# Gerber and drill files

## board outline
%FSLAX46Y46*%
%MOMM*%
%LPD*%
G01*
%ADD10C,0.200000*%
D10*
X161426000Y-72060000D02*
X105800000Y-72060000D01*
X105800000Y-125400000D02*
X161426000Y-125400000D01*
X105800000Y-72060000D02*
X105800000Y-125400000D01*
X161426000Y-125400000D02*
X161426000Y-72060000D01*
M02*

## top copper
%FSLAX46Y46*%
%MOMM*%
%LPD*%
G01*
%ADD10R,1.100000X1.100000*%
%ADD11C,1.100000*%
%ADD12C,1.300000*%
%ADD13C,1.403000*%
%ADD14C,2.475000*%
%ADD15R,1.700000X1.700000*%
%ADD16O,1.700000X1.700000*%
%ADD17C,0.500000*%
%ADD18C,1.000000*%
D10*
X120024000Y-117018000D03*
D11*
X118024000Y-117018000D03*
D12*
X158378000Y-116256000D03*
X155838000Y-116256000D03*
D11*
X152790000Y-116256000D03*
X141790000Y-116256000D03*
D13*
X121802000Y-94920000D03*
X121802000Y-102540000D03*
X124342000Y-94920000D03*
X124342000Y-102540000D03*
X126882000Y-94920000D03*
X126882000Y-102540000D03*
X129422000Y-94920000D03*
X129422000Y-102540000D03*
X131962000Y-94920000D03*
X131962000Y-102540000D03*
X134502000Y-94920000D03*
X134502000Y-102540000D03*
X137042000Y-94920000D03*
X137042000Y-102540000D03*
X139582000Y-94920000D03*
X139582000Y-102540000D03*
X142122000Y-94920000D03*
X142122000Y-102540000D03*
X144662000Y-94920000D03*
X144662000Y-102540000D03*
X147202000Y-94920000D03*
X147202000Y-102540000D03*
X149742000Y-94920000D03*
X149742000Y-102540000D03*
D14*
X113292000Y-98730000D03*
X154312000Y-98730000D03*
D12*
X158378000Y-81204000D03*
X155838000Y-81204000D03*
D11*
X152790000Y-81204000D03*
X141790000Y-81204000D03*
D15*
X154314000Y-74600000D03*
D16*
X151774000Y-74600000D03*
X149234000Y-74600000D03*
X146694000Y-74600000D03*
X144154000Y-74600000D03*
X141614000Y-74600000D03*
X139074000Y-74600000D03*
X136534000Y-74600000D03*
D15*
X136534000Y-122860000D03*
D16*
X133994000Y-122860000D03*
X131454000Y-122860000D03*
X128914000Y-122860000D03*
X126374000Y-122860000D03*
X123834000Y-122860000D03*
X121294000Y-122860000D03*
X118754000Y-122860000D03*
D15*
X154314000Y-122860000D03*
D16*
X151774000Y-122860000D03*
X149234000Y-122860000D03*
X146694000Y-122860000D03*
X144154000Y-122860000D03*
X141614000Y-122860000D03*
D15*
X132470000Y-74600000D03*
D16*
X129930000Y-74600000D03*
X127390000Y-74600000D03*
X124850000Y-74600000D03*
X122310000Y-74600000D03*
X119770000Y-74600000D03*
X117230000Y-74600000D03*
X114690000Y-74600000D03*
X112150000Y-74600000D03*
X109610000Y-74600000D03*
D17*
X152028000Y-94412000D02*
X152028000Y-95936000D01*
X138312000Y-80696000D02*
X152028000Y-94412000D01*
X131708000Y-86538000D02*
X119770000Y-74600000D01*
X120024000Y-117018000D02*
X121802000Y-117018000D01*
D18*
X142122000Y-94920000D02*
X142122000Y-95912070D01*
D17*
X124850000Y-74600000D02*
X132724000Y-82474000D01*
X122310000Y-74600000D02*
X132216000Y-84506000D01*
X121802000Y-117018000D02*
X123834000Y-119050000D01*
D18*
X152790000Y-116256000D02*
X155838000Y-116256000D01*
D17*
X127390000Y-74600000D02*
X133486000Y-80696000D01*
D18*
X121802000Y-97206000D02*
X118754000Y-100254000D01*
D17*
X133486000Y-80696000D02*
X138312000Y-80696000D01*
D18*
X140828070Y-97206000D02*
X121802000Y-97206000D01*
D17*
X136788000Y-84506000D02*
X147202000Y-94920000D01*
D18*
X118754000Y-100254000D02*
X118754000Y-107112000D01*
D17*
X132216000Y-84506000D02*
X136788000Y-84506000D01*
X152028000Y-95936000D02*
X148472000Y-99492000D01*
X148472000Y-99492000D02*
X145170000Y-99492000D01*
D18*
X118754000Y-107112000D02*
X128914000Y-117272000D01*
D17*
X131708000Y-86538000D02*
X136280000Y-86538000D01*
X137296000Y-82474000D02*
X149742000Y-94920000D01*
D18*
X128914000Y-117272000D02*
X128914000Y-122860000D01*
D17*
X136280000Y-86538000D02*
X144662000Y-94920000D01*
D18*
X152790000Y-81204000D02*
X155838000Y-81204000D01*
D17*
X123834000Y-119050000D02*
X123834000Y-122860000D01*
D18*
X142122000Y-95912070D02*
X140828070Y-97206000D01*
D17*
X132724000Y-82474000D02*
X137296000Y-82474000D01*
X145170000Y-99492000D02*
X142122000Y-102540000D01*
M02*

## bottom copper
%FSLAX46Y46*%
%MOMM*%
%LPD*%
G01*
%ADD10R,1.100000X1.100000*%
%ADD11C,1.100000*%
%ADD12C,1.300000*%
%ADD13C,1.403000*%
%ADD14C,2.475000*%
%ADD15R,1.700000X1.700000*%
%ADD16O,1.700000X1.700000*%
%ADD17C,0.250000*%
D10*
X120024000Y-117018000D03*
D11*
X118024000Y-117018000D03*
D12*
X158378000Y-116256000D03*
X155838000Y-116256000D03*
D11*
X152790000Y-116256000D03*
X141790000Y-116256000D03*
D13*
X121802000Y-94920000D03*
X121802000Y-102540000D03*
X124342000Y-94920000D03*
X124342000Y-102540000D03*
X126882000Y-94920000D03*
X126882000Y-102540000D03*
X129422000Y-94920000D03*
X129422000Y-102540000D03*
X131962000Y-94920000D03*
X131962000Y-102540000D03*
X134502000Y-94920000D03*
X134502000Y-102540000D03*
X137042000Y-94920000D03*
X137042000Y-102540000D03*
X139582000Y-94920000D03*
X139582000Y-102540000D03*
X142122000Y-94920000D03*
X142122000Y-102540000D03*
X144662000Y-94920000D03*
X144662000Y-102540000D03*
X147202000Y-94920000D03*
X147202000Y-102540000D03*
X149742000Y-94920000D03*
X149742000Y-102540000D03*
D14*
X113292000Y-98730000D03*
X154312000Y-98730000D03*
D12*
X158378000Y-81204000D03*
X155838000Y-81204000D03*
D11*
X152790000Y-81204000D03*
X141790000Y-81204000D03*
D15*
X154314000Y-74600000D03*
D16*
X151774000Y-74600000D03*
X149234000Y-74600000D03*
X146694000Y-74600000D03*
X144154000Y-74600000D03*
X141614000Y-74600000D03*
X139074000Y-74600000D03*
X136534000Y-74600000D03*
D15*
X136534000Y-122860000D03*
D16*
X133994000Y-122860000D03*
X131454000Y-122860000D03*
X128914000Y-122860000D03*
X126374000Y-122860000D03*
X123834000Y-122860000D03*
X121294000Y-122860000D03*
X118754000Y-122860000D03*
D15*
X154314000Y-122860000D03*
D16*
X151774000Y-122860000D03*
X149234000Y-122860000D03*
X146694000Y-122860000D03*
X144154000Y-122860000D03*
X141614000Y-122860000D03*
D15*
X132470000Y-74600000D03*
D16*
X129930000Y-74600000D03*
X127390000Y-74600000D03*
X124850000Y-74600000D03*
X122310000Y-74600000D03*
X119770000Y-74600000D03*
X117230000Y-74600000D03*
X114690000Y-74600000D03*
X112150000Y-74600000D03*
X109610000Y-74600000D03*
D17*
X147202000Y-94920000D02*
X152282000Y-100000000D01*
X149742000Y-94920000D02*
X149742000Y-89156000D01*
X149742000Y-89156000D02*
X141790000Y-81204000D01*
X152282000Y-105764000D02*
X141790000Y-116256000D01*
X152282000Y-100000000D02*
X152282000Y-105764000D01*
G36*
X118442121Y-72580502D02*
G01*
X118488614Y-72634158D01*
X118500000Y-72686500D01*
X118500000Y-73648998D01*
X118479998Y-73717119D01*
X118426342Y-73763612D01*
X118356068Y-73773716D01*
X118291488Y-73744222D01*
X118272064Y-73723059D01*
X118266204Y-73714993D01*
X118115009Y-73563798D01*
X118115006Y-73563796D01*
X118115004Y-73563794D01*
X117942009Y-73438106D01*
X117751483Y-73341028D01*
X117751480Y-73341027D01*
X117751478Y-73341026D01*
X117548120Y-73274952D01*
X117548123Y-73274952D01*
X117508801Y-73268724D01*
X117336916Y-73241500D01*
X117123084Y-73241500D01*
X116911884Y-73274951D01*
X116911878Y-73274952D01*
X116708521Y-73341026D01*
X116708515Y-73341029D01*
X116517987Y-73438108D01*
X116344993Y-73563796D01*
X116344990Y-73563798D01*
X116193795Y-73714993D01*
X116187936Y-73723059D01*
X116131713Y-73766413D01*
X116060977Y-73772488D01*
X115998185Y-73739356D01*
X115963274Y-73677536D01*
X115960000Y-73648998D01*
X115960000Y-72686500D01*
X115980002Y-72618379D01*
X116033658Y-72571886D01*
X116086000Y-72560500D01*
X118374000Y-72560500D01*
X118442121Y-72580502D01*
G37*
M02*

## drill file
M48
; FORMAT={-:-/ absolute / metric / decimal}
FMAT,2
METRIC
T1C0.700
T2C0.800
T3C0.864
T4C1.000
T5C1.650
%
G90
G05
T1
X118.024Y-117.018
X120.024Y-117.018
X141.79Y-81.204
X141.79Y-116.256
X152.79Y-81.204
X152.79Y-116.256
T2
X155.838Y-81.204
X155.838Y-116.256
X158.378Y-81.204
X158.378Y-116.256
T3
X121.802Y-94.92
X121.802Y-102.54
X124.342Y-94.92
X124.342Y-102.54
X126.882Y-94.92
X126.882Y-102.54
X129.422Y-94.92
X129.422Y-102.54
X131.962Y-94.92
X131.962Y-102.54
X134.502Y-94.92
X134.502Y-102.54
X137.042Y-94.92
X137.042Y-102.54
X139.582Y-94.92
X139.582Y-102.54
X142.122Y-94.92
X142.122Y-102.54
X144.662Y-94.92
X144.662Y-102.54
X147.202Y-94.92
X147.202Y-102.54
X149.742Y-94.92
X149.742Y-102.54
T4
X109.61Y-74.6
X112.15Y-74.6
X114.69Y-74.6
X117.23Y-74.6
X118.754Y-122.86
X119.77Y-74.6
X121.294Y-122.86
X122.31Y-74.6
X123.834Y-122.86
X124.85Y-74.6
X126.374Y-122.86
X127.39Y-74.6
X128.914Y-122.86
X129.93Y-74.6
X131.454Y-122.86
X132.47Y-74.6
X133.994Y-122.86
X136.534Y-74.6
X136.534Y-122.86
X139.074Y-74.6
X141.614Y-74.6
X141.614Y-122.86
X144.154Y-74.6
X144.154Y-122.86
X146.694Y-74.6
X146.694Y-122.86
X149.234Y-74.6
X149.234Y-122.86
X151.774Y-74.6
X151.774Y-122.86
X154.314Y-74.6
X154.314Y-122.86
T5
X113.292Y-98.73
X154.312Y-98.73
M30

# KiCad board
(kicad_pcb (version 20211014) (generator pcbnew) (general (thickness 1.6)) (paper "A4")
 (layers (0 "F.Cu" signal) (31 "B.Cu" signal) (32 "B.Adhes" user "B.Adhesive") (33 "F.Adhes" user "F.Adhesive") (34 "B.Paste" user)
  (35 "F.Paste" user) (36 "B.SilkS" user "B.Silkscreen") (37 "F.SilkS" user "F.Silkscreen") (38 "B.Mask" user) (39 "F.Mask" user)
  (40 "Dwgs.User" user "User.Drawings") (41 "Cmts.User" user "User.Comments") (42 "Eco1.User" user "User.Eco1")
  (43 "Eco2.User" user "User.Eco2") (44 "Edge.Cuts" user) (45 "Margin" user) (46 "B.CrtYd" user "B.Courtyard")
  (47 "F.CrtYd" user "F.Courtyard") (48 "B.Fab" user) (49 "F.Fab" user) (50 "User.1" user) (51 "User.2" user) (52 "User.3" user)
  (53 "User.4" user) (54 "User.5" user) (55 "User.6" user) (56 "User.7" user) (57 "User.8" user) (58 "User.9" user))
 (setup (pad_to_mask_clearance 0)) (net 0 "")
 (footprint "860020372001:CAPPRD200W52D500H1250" (layer "F.Cu") (at 120.024 117.018 180)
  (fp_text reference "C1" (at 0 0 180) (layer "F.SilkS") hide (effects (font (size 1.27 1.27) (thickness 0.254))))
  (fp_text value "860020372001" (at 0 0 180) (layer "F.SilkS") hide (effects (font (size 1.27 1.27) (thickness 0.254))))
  (pad "1" thru_hole rect locked (at 0 0 180) (size 1.1 1.1) (drill 0.7) (layers F&B.Cu *.Mask))
  (pad "2" thru_hole circle locked (at 2 0 180) (size 1.1 1.1) (drill 0.7) (layers F&B.Cu *.Mask)))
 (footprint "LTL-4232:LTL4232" (layer "F.Cu") (at 158.378 116.256 180)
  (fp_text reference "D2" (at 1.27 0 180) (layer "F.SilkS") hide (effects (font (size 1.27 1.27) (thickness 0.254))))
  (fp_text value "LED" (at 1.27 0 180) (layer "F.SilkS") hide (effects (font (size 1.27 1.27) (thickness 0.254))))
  (pad "1" thru_hole circle locked (at 0 0 180) (size 1.3 1.3) (drill 0.8) (layers F&B.Cu *.Mask))
  (pad "2" thru_hole circle locked (at 2.54 0 180) (size 1.3 1.3) (drill 0.8) (layers F&B.Cu *.Mask)))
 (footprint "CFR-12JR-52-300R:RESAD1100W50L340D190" (layer "F.Cu") (at 152.79 116.256 180)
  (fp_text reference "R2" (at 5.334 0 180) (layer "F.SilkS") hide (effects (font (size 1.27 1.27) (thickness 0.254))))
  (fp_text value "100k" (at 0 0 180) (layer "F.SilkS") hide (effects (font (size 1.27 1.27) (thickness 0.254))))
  (pad "1" thru_hole circle locked (at 0 0 180) (size 1.1 1.1) (drill 0.7) (layers F&B.Cu *.Mask))
  (pad "2" thru_hole circle locked (at 11 0 180) (size 1.1 1.1) (drill 0.7) (layers F&B.Cu *.Mask)))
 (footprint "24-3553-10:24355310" (layer "F.Cu") (at 121.802 94.92)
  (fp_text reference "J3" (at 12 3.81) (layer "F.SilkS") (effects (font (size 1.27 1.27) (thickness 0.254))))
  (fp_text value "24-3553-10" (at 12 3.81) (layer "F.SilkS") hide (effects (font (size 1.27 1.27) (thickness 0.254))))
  (pad "1" thru_hole circle locked (at 0 0) (size 1.403 1.403) (drill 0.8636) (layers F&B.Cu *.Mask))
  (pad "2" thru_hole circle locked (at 0 7.62) (size 1.403 1.403) (drill 0.8636) (layers F&B.Cu *.Mask))
  (pad "3" thru_hole circle locked (at 2.54 0) (size 1.403 1.403) (drill 0.8636) (layers F&B.Cu *.Mask))
  (pad "4" thru_hole circle locked (at 2.54 7.62) (size 1.403 1.403) (drill 0.8636) (layers F&B.Cu *.Mask))
  (pad "5" thru_hole circle locked (at 5.08 0) (size 1.403 1.403) (drill 0.8636) (layers F&B.Cu *.Mask))
  (pad "6" thru_hole circle locked (at 5.08 7.62) (size 1.403 1.403) (drill 0.8636) (layers F&B.Cu *.Mask))
  (pad "7" thru_hole circle locked (at 7.62 0) (size 1.403 1.403) (drill 0.8636) (layers F&B.Cu *.Mask))
  (pad "8" thru_hole circle locked (at 7.62 7.62) (size 1.403 1.403) (drill 0.8636) (layers F&B.Cu *.Mask))
  (pad "9" thru_hole circle locked (at 10.16 0) (size 1.403 1.403) (drill 0.8636) (layers F&B.Cu *.Mask))
  (pad "10" thru_hole circle locked (at 10.16 7.62) (size 1.403 1.403) (drill 0.8636) (layers F&B.Cu *.Mask))
  (pad "11" thru_hole circle locked (at 12.7 0) (size 1.403 1.403) (drill 0.8636) (layers F&B.Cu *.Mask))
  (pad "12" thru_hole circle locked (at 12.7 7.62) (size 1.403 1.403) (drill 0.8636) (layers F&B.Cu *.Mask))
  (pad "13" thru_hole circle locked (at 15.24 0) (size 1.403 1.403) (drill 0.8636) (layers F&B.Cu *.Mask))
  (pad "14" thru_hole circle locked (at 15.24 7.62) (size 1.403 1.403) (drill 0.8636) (layers F&B.Cu *.Mask))
  (pad "15" thru_hole circle locked (at 17.78 0) (size 1.403 1.403) (drill 0.8636) (layers F&B.Cu *.Mask))
  (pad "16" thru_hole circle locked (at 17.78 7.62) (size 1.403 1.403) (drill 0.8636) (layers F&B.Cu *.Mask))
  (pad "17" thru_hole circle locked (at 20.32 0) (size 1.403 1.403) (drill 0.8636) (layers F&B.Cu *.Mask))
  (pad "18" thru_hole circle locked (at 20.32 7.62) (size 1.403 1.403) (drill 0.8636) (layers F&B.Cu *.Mask))
  (pad "19" thru_hole circle locked (at 22.86 0) (size 1.403 1.403) (drill 0.8636) (layers F&B.Cu *.Mask))
  (pad "20" thru_hole circle locked (at 22.86 7.62) (size 1.403 1.403) (drill 0.8636) (layers F&B.Cu *.Mask))
  (pad "21" thru_hole circle locked (at 25.4 0) (size 1.403 1.403) (drill 0.8636) (layers F&B.Cu *.Mask))
  (pad "22" thru_hole circle locked (at 25.4 7.62) (size 1.403 1.403) (drill 0.8636) (layers F&B.Cu *.Mask))
  (pad "23" thru_hole circle locked (at 27.94 0) (size 1.403 1.403) (drill 0.8636) (layers F&B.Cu *.Mask))
  (pad "24" thru_hole circle locked (at 27.94 7.62) (size 1.403 1.403) (drill 0.8636) (layers F&B.Cu *.Mask))
  (pad "MH1" thru_hole circle locked (at -8.51 3.81) (size 2.475 2.475) (drill 1.65) (layers F&B.Cu *.Mask))
  (pad "MH2" thru_hole circle locked (at 32.51 3.81) (size 2.475 2.475) (drill 1.65) (layers F&B.Cu *.Mask)))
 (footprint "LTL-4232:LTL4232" (layer "F.Cu") (at 158.378 81.204 180)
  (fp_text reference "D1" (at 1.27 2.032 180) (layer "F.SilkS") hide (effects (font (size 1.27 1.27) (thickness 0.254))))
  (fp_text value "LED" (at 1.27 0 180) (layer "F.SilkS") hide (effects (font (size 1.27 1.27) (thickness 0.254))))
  (pad "1" thru_hole circle locked (at 0 0 180) (size 1.3 1.3) (drill 0.8) (layers F&B.Cu *.Mask))
  (pad "2" thru_hole circle locked (at 2.54 0 180) (size 1.3 1.3) (drill 0.8) (layers F&B.Cu *.Mask)))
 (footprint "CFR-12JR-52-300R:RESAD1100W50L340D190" (layer "F.Cu") (at 152.79 81.204 180)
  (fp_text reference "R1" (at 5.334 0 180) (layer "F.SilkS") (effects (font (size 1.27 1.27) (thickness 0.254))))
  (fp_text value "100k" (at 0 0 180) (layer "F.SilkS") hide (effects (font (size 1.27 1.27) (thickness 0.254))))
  (pad "1" thru_hole circle locked (at 0 0 180) (size 1.1 1.1) (drill 0.7) (layers F&B.Cu *.Mask))
  (pad "2" thru_hole circle locked (at 11 0 180) (size 1.1 1.1) (drill 0.7) (layers F&B.Cu *.Mask)))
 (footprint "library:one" (layer "B.Cu") (at 135.01 90.094)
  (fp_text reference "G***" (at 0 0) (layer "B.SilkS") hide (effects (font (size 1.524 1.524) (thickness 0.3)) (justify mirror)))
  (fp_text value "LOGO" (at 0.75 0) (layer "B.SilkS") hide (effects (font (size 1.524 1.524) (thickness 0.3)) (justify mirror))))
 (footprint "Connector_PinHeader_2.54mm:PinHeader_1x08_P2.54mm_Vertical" (layer "B.Cu") (at 154.314 74.6 90)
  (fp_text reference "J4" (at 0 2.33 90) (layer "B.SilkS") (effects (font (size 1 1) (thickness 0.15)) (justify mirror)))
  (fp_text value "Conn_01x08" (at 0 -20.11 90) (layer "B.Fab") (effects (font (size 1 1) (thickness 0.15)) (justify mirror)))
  (pad "1" thru_hole rect locked (at 0 0 90) (size 1.7 1.7) (drill 1) (layers F&B.Cu *.Mask))
  (pad "2" thru_hole oval locked (at 0 -2.54 90) (size 1.7 1.7) (drill 1) (layers F&B.Cu *.Mask))
  (pad "3" thru_hole oval locked (at 0 -5.08 90) (size 1.7 1.7) (drill 1) (layers F&B.Cu *.Mask))
  (pad "4" thru_hole oval locked (at 0 -7.62 90) (size 1.7 1.7) (drill 1) (layers F&B.Cu *.Mask))
  (pad "5" thru_hole oval locked (at 0 -10.16 90) (size 1.7 1.7) (drill 1) (layers F&B.Cu *.Mask))
  (pad "6" thru_hole oval locked (at 0 -12.7 90) (size 1.7 1.7) (drill 1) (layers F&B.Cu *.Mask))
  (pad "7" thru_hole oval locked (at 0 -15.24 90) (size 1.7 1.7) (drill 1) (layers F&B.Cu *.Mask))
  (pad "8" thru_hole oval locked (at 0 -17.78 90) (size 1.7 1.7) (drill 1) (layers F&B.Cu *.Mask)))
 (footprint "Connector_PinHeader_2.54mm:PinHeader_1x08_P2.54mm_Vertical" (layer "B.Cu") (at 136.534 122.86 90)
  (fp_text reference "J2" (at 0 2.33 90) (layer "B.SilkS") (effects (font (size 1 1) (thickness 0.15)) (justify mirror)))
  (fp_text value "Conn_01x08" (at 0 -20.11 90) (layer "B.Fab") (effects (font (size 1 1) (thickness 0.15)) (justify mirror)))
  (pad "1" thru_hole rect locked (at 0 0 90) (size 1.7 1.7) (drill 1) (layers F&B.Cu *.Mask))
  (pad "2" thru_hole oval locked (at 0 -2.54 90) (size 1.7 1.7) (drill 1) (layers F&B.Cu *.Mask))
  (pad "3" thru_hole oval locked (at 0 -5.08 90) (size 1.7 1.7) (drill 1) (layers F&B.Cu *.Mask))
  (pad "4" thru_hole oval locked (at 0 -7.62 90) (size 1.7 1.7) (drill 1) (layers F&B.Cu *.Mask))
  (pad "5" thru_hole oval locked (at 0 -10.16 90) (size 1.7 1.7) (drill 1) (layers F&B.Cu *.Mask))
  (pad "6" thru_hole oval locked (at 0 -12.7 90) (size 1.7 1.7) (drill 1) (layers F&B.Cu *.Mask))
  (pad "7" thru_hole oval locked (at 0 -15.24 90) (size 1.7 1.7) (drill 1) (layers F&B.Cu *.Mask))
  (pad "8" thru_hole oval locked (at 0 -17.78 90) (size 1.7 1.7) (drill 1) (layers F&B.Cu *.Mask)))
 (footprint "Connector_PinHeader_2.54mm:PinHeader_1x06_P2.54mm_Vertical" (layer "B.Cu") (at 154.314 122.86 90)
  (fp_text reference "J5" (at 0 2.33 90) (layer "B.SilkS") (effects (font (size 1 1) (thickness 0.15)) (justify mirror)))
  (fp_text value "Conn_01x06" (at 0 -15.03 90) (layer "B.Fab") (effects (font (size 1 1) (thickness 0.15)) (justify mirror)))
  (pad "1" thru_hole rect locked (at 0 0 90) (size 1.7 1.7) (drill 1) (layers F&B.Cu *.Mask))
  (pad "2" thru_hole oval locked (at 0 -2.54 90) (size 1.7 1.7) (drill 1) (layers F&B.Cu *.Mask))
  (pad "3" thru_hole oval locked (at 0 -5.08 90) (size 1.7 1.7) (drill 1) (layers F&B.Cu *.Mask))
  (pad "4" thru_hole oval locked (at 0 -7.62 90) (size 1.7 1.7) (drill 1) (layers F&B.Cu *.Mask))
  (pad "5" thru_hole oval locked (at 0 -10.16 90) (size 1.7 1.7) (drill 1) (layers F&B.Cu *.Mask))
  (pad "6" thru_hole oval locked (at 0 -12.7 90) (size 1.7 1.7) (drill 1) (layers F&B.Cu *.Mask)))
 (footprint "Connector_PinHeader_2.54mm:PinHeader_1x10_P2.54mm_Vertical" (layer "B.Cu") (at 132.47 74.6 90)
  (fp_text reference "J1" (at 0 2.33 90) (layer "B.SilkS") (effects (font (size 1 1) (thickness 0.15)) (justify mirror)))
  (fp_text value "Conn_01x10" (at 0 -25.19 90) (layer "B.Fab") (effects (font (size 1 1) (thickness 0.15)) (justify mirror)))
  (pad "1" thru_hole rect locked (at 0 0 90) (size 1.7 1.7) (drill 1) (layers F&B.Cu *.Mask))
  (pad "2" thru_hole oval locked (at 0 -2.54 90) (size 1.7 1.7) (drill 1) (layers F&B.Cu *.Mask))
  (pad "3" thru_hole oval locked (at 0 -5.08 90) (size 1.7 1.7) (drill 1) (layers F&B.Cu *.Mask))
  (pad "4" thru_hole oval locked (at 0 -7.62 90) (size 1.7 1.7) (drill 1) (layers F&B.Cu *.Mask))
  (pad "5" thru_hole oval locked (at 0 -10.16 90) (size 1.7 1.7) (drill 1) (layers F&B.Cu *.Mask))
  (pad "6" thru_hole oval locked (at 0 -12.7 90) (size 1.7 1.7) (drill 1) (layers F&B.Cu *.Mask))
  (pad "7" thru_hole oval locked (at 0 -15.24 90) (size 1.7 1.7) (drill 1) (layers F&B.Cu *.Mask))
  (pad "8" thru_hole oval locked (at 0 -17.78 90) (size 1.7 1.7) (drill 1) (layers F&B.Cu *.Mask))
  (pad "9" thru_hole oval locked (at 0 -20.32 90) (size 1.7 1.7) (drill 1) (layers F&B.Cu *.Mask))
  (pad "10" thru_hole oval locked (at 0 -22.86 90) (size 1.7 1.7) (drill 1) (layers F&B.Cu *.Mask)))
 (gr_line (start 161.426 72.06) (end 105.8 72.06) (layer "Edge.Cuts") (width 0.2))
 (gr_line (start 105.8 125.4) (end 161.426 125.4) (layer "Edge.Cuts") (width 0.2))
 (gr_line (start 105.8 72.06) (end 105.8 125.4) (layer "Edge.Cuts") (width 0.2))
 (gr_line (start 161.426 125.4) (end 161.426 72.06) (layer "Edge.Cuts") (width 0.2))
 (segment (start 152.028 94.412) (end 152.028 95.936) (width 0.5) (layer "F.Cu") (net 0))
 (segment (start 138.312 80.696) (end 152.028 94.412) (width 0.5) (layer "F.Cu") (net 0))
 (segment (start 131.708 86.538) (end 119.77 74.6) (width 0.5) (layer "F.Cu") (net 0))
 (segment (start 120.024 117.018) (end 121.802 117.018) (width 0.5) (layer "F.Cu") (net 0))
 (segment (start 142.122 94.92) (end 142.122 95.91207) (width 1) (layer "F.Cu") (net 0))
 (segment (start 124.85 74.6) (end 132.724 82.474) (width 0.5) (layer "F.Cu") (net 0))
 (segment (start 122.31 74.6) (end 132.216 84.506) (width 0.5) (layer "F.Cu") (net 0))
 (segment (start 121.802 117.018) (end 123.834 119.05) (width 0.5) (layer "F.Cu") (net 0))
 (segment (start 152.79 116.256) (end 155.838 116.256) (width 1) (layer "F.Cu") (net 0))
 (segment (start 127.39 74.6) (end 133.486 80.696) (width 0.5) (layer "F.Cu") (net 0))
 (segment (start 121.802 97.206) (end 118.754 100.254) (width 1) (layer "F.Cu") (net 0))
 (segment (start 133.486 80.696) (end 138.312 80.696) (width 0.5) (layer "F.Cu") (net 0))
 (segment (start 140.82807 97.206) (end 121.802 97.206) (width 1) (layer "F.Cu") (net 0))
 (segment (start 136.788 84.506) (end 147.202 94.92) (width 0.5) (layer "F.Cu") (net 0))
 (segment (start 118.754 100.254) (end 118.754 107.112) (width 1) (layer "F.Cu") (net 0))
 (segment (start 132.216 84.506) (end 136.788 84.506) (width 0.5) (layer "F.Cu") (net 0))
 (segment (start 152.028 95.936) (end 148.472 99.492) (width 0.5) (layer "F.Cu") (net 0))
 (segment (start 148.472 99.492) (end 145.17 99.492) (width 0.5) (layer "F.Cu") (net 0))
 (segment (start 118.754 107.112) (end 128.914 117.272) (width 1) (layer "F.Cu") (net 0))
 (segment (start 131.708 86.538) (end 136.28 86.538) (width 0.5) (layer "F.Cu") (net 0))
 (segment (start 137.296 82.474) (end 149.742 94.92) (width 0.5) (layer "F.Cu") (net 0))
 (segment (start 128.914 117.272) (end 128.914 122.86) (width 1) (layer "F.Cu") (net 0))
 (segment (start 136.28 86.538) (end 144.662 94.92) (width 0.5) (layer "F.Cu") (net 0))
 (segment (start 152.79 81.204) (end 155.838 81.204) (width 1) (layer "F.Cu") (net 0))
 (segment (start 123.834 119.05) (end 123.834 122.86) (width 0.5) (layer "F.Cu") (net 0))
 (segment (start 142.122 95.91207) (end 140.82807 97.206) (width 1) (layer "F.Cu") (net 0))
 (segment (start 132.724 82.474) (end 137.296 82.474) (width 0.5) (layer "F.Cu") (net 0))
 (segment (start 145.17 99.492) (end 142.122 102.54) (width 0.5) (layer "F.Cu") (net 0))
 (segment (start 147.202 94.92) (end 152.282 100) (width 0.25) (layer "B.Cu") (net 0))
 (segment (start 149.742 94.92) (end 149.742 89.156) (width 0.25) (layer "B.Cu") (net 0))
 (segment (start 149.742 89.156) (end 141.79 81.204) (width 0.25) (layer "B.Cu") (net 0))
 (segment (start 152.282 105.764) (end 141.79 116.256) (width 0.25) (layer "B.Cu") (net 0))
 (segment (start 152.282 100) (end 152.282 105.764) (width 0.25) (layer "B.Cu") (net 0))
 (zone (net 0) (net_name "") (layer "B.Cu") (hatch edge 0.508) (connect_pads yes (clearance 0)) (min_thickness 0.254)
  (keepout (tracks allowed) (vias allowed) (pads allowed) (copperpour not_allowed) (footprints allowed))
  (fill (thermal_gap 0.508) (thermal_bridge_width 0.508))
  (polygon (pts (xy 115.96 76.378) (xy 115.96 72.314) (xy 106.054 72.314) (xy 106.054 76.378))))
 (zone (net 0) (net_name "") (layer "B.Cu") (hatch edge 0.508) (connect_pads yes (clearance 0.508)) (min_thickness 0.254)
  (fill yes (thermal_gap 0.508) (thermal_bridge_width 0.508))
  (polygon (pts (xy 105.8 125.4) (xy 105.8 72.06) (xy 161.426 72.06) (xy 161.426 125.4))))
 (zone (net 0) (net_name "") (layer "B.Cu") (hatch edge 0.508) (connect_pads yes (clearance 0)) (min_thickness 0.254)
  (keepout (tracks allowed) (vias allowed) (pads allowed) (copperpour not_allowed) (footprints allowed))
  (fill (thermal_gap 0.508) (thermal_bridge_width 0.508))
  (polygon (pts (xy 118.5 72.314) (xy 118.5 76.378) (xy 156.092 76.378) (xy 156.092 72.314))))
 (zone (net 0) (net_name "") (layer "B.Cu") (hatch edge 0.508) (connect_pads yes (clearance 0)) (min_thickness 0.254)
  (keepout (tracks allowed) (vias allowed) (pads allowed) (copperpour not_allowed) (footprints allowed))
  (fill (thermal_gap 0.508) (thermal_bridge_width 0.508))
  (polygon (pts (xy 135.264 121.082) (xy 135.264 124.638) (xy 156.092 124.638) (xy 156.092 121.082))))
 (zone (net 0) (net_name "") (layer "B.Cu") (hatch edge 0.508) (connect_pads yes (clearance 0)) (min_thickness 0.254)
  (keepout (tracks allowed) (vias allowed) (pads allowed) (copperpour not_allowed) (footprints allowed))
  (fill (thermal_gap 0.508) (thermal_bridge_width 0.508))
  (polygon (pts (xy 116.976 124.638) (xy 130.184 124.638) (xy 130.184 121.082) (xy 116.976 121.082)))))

